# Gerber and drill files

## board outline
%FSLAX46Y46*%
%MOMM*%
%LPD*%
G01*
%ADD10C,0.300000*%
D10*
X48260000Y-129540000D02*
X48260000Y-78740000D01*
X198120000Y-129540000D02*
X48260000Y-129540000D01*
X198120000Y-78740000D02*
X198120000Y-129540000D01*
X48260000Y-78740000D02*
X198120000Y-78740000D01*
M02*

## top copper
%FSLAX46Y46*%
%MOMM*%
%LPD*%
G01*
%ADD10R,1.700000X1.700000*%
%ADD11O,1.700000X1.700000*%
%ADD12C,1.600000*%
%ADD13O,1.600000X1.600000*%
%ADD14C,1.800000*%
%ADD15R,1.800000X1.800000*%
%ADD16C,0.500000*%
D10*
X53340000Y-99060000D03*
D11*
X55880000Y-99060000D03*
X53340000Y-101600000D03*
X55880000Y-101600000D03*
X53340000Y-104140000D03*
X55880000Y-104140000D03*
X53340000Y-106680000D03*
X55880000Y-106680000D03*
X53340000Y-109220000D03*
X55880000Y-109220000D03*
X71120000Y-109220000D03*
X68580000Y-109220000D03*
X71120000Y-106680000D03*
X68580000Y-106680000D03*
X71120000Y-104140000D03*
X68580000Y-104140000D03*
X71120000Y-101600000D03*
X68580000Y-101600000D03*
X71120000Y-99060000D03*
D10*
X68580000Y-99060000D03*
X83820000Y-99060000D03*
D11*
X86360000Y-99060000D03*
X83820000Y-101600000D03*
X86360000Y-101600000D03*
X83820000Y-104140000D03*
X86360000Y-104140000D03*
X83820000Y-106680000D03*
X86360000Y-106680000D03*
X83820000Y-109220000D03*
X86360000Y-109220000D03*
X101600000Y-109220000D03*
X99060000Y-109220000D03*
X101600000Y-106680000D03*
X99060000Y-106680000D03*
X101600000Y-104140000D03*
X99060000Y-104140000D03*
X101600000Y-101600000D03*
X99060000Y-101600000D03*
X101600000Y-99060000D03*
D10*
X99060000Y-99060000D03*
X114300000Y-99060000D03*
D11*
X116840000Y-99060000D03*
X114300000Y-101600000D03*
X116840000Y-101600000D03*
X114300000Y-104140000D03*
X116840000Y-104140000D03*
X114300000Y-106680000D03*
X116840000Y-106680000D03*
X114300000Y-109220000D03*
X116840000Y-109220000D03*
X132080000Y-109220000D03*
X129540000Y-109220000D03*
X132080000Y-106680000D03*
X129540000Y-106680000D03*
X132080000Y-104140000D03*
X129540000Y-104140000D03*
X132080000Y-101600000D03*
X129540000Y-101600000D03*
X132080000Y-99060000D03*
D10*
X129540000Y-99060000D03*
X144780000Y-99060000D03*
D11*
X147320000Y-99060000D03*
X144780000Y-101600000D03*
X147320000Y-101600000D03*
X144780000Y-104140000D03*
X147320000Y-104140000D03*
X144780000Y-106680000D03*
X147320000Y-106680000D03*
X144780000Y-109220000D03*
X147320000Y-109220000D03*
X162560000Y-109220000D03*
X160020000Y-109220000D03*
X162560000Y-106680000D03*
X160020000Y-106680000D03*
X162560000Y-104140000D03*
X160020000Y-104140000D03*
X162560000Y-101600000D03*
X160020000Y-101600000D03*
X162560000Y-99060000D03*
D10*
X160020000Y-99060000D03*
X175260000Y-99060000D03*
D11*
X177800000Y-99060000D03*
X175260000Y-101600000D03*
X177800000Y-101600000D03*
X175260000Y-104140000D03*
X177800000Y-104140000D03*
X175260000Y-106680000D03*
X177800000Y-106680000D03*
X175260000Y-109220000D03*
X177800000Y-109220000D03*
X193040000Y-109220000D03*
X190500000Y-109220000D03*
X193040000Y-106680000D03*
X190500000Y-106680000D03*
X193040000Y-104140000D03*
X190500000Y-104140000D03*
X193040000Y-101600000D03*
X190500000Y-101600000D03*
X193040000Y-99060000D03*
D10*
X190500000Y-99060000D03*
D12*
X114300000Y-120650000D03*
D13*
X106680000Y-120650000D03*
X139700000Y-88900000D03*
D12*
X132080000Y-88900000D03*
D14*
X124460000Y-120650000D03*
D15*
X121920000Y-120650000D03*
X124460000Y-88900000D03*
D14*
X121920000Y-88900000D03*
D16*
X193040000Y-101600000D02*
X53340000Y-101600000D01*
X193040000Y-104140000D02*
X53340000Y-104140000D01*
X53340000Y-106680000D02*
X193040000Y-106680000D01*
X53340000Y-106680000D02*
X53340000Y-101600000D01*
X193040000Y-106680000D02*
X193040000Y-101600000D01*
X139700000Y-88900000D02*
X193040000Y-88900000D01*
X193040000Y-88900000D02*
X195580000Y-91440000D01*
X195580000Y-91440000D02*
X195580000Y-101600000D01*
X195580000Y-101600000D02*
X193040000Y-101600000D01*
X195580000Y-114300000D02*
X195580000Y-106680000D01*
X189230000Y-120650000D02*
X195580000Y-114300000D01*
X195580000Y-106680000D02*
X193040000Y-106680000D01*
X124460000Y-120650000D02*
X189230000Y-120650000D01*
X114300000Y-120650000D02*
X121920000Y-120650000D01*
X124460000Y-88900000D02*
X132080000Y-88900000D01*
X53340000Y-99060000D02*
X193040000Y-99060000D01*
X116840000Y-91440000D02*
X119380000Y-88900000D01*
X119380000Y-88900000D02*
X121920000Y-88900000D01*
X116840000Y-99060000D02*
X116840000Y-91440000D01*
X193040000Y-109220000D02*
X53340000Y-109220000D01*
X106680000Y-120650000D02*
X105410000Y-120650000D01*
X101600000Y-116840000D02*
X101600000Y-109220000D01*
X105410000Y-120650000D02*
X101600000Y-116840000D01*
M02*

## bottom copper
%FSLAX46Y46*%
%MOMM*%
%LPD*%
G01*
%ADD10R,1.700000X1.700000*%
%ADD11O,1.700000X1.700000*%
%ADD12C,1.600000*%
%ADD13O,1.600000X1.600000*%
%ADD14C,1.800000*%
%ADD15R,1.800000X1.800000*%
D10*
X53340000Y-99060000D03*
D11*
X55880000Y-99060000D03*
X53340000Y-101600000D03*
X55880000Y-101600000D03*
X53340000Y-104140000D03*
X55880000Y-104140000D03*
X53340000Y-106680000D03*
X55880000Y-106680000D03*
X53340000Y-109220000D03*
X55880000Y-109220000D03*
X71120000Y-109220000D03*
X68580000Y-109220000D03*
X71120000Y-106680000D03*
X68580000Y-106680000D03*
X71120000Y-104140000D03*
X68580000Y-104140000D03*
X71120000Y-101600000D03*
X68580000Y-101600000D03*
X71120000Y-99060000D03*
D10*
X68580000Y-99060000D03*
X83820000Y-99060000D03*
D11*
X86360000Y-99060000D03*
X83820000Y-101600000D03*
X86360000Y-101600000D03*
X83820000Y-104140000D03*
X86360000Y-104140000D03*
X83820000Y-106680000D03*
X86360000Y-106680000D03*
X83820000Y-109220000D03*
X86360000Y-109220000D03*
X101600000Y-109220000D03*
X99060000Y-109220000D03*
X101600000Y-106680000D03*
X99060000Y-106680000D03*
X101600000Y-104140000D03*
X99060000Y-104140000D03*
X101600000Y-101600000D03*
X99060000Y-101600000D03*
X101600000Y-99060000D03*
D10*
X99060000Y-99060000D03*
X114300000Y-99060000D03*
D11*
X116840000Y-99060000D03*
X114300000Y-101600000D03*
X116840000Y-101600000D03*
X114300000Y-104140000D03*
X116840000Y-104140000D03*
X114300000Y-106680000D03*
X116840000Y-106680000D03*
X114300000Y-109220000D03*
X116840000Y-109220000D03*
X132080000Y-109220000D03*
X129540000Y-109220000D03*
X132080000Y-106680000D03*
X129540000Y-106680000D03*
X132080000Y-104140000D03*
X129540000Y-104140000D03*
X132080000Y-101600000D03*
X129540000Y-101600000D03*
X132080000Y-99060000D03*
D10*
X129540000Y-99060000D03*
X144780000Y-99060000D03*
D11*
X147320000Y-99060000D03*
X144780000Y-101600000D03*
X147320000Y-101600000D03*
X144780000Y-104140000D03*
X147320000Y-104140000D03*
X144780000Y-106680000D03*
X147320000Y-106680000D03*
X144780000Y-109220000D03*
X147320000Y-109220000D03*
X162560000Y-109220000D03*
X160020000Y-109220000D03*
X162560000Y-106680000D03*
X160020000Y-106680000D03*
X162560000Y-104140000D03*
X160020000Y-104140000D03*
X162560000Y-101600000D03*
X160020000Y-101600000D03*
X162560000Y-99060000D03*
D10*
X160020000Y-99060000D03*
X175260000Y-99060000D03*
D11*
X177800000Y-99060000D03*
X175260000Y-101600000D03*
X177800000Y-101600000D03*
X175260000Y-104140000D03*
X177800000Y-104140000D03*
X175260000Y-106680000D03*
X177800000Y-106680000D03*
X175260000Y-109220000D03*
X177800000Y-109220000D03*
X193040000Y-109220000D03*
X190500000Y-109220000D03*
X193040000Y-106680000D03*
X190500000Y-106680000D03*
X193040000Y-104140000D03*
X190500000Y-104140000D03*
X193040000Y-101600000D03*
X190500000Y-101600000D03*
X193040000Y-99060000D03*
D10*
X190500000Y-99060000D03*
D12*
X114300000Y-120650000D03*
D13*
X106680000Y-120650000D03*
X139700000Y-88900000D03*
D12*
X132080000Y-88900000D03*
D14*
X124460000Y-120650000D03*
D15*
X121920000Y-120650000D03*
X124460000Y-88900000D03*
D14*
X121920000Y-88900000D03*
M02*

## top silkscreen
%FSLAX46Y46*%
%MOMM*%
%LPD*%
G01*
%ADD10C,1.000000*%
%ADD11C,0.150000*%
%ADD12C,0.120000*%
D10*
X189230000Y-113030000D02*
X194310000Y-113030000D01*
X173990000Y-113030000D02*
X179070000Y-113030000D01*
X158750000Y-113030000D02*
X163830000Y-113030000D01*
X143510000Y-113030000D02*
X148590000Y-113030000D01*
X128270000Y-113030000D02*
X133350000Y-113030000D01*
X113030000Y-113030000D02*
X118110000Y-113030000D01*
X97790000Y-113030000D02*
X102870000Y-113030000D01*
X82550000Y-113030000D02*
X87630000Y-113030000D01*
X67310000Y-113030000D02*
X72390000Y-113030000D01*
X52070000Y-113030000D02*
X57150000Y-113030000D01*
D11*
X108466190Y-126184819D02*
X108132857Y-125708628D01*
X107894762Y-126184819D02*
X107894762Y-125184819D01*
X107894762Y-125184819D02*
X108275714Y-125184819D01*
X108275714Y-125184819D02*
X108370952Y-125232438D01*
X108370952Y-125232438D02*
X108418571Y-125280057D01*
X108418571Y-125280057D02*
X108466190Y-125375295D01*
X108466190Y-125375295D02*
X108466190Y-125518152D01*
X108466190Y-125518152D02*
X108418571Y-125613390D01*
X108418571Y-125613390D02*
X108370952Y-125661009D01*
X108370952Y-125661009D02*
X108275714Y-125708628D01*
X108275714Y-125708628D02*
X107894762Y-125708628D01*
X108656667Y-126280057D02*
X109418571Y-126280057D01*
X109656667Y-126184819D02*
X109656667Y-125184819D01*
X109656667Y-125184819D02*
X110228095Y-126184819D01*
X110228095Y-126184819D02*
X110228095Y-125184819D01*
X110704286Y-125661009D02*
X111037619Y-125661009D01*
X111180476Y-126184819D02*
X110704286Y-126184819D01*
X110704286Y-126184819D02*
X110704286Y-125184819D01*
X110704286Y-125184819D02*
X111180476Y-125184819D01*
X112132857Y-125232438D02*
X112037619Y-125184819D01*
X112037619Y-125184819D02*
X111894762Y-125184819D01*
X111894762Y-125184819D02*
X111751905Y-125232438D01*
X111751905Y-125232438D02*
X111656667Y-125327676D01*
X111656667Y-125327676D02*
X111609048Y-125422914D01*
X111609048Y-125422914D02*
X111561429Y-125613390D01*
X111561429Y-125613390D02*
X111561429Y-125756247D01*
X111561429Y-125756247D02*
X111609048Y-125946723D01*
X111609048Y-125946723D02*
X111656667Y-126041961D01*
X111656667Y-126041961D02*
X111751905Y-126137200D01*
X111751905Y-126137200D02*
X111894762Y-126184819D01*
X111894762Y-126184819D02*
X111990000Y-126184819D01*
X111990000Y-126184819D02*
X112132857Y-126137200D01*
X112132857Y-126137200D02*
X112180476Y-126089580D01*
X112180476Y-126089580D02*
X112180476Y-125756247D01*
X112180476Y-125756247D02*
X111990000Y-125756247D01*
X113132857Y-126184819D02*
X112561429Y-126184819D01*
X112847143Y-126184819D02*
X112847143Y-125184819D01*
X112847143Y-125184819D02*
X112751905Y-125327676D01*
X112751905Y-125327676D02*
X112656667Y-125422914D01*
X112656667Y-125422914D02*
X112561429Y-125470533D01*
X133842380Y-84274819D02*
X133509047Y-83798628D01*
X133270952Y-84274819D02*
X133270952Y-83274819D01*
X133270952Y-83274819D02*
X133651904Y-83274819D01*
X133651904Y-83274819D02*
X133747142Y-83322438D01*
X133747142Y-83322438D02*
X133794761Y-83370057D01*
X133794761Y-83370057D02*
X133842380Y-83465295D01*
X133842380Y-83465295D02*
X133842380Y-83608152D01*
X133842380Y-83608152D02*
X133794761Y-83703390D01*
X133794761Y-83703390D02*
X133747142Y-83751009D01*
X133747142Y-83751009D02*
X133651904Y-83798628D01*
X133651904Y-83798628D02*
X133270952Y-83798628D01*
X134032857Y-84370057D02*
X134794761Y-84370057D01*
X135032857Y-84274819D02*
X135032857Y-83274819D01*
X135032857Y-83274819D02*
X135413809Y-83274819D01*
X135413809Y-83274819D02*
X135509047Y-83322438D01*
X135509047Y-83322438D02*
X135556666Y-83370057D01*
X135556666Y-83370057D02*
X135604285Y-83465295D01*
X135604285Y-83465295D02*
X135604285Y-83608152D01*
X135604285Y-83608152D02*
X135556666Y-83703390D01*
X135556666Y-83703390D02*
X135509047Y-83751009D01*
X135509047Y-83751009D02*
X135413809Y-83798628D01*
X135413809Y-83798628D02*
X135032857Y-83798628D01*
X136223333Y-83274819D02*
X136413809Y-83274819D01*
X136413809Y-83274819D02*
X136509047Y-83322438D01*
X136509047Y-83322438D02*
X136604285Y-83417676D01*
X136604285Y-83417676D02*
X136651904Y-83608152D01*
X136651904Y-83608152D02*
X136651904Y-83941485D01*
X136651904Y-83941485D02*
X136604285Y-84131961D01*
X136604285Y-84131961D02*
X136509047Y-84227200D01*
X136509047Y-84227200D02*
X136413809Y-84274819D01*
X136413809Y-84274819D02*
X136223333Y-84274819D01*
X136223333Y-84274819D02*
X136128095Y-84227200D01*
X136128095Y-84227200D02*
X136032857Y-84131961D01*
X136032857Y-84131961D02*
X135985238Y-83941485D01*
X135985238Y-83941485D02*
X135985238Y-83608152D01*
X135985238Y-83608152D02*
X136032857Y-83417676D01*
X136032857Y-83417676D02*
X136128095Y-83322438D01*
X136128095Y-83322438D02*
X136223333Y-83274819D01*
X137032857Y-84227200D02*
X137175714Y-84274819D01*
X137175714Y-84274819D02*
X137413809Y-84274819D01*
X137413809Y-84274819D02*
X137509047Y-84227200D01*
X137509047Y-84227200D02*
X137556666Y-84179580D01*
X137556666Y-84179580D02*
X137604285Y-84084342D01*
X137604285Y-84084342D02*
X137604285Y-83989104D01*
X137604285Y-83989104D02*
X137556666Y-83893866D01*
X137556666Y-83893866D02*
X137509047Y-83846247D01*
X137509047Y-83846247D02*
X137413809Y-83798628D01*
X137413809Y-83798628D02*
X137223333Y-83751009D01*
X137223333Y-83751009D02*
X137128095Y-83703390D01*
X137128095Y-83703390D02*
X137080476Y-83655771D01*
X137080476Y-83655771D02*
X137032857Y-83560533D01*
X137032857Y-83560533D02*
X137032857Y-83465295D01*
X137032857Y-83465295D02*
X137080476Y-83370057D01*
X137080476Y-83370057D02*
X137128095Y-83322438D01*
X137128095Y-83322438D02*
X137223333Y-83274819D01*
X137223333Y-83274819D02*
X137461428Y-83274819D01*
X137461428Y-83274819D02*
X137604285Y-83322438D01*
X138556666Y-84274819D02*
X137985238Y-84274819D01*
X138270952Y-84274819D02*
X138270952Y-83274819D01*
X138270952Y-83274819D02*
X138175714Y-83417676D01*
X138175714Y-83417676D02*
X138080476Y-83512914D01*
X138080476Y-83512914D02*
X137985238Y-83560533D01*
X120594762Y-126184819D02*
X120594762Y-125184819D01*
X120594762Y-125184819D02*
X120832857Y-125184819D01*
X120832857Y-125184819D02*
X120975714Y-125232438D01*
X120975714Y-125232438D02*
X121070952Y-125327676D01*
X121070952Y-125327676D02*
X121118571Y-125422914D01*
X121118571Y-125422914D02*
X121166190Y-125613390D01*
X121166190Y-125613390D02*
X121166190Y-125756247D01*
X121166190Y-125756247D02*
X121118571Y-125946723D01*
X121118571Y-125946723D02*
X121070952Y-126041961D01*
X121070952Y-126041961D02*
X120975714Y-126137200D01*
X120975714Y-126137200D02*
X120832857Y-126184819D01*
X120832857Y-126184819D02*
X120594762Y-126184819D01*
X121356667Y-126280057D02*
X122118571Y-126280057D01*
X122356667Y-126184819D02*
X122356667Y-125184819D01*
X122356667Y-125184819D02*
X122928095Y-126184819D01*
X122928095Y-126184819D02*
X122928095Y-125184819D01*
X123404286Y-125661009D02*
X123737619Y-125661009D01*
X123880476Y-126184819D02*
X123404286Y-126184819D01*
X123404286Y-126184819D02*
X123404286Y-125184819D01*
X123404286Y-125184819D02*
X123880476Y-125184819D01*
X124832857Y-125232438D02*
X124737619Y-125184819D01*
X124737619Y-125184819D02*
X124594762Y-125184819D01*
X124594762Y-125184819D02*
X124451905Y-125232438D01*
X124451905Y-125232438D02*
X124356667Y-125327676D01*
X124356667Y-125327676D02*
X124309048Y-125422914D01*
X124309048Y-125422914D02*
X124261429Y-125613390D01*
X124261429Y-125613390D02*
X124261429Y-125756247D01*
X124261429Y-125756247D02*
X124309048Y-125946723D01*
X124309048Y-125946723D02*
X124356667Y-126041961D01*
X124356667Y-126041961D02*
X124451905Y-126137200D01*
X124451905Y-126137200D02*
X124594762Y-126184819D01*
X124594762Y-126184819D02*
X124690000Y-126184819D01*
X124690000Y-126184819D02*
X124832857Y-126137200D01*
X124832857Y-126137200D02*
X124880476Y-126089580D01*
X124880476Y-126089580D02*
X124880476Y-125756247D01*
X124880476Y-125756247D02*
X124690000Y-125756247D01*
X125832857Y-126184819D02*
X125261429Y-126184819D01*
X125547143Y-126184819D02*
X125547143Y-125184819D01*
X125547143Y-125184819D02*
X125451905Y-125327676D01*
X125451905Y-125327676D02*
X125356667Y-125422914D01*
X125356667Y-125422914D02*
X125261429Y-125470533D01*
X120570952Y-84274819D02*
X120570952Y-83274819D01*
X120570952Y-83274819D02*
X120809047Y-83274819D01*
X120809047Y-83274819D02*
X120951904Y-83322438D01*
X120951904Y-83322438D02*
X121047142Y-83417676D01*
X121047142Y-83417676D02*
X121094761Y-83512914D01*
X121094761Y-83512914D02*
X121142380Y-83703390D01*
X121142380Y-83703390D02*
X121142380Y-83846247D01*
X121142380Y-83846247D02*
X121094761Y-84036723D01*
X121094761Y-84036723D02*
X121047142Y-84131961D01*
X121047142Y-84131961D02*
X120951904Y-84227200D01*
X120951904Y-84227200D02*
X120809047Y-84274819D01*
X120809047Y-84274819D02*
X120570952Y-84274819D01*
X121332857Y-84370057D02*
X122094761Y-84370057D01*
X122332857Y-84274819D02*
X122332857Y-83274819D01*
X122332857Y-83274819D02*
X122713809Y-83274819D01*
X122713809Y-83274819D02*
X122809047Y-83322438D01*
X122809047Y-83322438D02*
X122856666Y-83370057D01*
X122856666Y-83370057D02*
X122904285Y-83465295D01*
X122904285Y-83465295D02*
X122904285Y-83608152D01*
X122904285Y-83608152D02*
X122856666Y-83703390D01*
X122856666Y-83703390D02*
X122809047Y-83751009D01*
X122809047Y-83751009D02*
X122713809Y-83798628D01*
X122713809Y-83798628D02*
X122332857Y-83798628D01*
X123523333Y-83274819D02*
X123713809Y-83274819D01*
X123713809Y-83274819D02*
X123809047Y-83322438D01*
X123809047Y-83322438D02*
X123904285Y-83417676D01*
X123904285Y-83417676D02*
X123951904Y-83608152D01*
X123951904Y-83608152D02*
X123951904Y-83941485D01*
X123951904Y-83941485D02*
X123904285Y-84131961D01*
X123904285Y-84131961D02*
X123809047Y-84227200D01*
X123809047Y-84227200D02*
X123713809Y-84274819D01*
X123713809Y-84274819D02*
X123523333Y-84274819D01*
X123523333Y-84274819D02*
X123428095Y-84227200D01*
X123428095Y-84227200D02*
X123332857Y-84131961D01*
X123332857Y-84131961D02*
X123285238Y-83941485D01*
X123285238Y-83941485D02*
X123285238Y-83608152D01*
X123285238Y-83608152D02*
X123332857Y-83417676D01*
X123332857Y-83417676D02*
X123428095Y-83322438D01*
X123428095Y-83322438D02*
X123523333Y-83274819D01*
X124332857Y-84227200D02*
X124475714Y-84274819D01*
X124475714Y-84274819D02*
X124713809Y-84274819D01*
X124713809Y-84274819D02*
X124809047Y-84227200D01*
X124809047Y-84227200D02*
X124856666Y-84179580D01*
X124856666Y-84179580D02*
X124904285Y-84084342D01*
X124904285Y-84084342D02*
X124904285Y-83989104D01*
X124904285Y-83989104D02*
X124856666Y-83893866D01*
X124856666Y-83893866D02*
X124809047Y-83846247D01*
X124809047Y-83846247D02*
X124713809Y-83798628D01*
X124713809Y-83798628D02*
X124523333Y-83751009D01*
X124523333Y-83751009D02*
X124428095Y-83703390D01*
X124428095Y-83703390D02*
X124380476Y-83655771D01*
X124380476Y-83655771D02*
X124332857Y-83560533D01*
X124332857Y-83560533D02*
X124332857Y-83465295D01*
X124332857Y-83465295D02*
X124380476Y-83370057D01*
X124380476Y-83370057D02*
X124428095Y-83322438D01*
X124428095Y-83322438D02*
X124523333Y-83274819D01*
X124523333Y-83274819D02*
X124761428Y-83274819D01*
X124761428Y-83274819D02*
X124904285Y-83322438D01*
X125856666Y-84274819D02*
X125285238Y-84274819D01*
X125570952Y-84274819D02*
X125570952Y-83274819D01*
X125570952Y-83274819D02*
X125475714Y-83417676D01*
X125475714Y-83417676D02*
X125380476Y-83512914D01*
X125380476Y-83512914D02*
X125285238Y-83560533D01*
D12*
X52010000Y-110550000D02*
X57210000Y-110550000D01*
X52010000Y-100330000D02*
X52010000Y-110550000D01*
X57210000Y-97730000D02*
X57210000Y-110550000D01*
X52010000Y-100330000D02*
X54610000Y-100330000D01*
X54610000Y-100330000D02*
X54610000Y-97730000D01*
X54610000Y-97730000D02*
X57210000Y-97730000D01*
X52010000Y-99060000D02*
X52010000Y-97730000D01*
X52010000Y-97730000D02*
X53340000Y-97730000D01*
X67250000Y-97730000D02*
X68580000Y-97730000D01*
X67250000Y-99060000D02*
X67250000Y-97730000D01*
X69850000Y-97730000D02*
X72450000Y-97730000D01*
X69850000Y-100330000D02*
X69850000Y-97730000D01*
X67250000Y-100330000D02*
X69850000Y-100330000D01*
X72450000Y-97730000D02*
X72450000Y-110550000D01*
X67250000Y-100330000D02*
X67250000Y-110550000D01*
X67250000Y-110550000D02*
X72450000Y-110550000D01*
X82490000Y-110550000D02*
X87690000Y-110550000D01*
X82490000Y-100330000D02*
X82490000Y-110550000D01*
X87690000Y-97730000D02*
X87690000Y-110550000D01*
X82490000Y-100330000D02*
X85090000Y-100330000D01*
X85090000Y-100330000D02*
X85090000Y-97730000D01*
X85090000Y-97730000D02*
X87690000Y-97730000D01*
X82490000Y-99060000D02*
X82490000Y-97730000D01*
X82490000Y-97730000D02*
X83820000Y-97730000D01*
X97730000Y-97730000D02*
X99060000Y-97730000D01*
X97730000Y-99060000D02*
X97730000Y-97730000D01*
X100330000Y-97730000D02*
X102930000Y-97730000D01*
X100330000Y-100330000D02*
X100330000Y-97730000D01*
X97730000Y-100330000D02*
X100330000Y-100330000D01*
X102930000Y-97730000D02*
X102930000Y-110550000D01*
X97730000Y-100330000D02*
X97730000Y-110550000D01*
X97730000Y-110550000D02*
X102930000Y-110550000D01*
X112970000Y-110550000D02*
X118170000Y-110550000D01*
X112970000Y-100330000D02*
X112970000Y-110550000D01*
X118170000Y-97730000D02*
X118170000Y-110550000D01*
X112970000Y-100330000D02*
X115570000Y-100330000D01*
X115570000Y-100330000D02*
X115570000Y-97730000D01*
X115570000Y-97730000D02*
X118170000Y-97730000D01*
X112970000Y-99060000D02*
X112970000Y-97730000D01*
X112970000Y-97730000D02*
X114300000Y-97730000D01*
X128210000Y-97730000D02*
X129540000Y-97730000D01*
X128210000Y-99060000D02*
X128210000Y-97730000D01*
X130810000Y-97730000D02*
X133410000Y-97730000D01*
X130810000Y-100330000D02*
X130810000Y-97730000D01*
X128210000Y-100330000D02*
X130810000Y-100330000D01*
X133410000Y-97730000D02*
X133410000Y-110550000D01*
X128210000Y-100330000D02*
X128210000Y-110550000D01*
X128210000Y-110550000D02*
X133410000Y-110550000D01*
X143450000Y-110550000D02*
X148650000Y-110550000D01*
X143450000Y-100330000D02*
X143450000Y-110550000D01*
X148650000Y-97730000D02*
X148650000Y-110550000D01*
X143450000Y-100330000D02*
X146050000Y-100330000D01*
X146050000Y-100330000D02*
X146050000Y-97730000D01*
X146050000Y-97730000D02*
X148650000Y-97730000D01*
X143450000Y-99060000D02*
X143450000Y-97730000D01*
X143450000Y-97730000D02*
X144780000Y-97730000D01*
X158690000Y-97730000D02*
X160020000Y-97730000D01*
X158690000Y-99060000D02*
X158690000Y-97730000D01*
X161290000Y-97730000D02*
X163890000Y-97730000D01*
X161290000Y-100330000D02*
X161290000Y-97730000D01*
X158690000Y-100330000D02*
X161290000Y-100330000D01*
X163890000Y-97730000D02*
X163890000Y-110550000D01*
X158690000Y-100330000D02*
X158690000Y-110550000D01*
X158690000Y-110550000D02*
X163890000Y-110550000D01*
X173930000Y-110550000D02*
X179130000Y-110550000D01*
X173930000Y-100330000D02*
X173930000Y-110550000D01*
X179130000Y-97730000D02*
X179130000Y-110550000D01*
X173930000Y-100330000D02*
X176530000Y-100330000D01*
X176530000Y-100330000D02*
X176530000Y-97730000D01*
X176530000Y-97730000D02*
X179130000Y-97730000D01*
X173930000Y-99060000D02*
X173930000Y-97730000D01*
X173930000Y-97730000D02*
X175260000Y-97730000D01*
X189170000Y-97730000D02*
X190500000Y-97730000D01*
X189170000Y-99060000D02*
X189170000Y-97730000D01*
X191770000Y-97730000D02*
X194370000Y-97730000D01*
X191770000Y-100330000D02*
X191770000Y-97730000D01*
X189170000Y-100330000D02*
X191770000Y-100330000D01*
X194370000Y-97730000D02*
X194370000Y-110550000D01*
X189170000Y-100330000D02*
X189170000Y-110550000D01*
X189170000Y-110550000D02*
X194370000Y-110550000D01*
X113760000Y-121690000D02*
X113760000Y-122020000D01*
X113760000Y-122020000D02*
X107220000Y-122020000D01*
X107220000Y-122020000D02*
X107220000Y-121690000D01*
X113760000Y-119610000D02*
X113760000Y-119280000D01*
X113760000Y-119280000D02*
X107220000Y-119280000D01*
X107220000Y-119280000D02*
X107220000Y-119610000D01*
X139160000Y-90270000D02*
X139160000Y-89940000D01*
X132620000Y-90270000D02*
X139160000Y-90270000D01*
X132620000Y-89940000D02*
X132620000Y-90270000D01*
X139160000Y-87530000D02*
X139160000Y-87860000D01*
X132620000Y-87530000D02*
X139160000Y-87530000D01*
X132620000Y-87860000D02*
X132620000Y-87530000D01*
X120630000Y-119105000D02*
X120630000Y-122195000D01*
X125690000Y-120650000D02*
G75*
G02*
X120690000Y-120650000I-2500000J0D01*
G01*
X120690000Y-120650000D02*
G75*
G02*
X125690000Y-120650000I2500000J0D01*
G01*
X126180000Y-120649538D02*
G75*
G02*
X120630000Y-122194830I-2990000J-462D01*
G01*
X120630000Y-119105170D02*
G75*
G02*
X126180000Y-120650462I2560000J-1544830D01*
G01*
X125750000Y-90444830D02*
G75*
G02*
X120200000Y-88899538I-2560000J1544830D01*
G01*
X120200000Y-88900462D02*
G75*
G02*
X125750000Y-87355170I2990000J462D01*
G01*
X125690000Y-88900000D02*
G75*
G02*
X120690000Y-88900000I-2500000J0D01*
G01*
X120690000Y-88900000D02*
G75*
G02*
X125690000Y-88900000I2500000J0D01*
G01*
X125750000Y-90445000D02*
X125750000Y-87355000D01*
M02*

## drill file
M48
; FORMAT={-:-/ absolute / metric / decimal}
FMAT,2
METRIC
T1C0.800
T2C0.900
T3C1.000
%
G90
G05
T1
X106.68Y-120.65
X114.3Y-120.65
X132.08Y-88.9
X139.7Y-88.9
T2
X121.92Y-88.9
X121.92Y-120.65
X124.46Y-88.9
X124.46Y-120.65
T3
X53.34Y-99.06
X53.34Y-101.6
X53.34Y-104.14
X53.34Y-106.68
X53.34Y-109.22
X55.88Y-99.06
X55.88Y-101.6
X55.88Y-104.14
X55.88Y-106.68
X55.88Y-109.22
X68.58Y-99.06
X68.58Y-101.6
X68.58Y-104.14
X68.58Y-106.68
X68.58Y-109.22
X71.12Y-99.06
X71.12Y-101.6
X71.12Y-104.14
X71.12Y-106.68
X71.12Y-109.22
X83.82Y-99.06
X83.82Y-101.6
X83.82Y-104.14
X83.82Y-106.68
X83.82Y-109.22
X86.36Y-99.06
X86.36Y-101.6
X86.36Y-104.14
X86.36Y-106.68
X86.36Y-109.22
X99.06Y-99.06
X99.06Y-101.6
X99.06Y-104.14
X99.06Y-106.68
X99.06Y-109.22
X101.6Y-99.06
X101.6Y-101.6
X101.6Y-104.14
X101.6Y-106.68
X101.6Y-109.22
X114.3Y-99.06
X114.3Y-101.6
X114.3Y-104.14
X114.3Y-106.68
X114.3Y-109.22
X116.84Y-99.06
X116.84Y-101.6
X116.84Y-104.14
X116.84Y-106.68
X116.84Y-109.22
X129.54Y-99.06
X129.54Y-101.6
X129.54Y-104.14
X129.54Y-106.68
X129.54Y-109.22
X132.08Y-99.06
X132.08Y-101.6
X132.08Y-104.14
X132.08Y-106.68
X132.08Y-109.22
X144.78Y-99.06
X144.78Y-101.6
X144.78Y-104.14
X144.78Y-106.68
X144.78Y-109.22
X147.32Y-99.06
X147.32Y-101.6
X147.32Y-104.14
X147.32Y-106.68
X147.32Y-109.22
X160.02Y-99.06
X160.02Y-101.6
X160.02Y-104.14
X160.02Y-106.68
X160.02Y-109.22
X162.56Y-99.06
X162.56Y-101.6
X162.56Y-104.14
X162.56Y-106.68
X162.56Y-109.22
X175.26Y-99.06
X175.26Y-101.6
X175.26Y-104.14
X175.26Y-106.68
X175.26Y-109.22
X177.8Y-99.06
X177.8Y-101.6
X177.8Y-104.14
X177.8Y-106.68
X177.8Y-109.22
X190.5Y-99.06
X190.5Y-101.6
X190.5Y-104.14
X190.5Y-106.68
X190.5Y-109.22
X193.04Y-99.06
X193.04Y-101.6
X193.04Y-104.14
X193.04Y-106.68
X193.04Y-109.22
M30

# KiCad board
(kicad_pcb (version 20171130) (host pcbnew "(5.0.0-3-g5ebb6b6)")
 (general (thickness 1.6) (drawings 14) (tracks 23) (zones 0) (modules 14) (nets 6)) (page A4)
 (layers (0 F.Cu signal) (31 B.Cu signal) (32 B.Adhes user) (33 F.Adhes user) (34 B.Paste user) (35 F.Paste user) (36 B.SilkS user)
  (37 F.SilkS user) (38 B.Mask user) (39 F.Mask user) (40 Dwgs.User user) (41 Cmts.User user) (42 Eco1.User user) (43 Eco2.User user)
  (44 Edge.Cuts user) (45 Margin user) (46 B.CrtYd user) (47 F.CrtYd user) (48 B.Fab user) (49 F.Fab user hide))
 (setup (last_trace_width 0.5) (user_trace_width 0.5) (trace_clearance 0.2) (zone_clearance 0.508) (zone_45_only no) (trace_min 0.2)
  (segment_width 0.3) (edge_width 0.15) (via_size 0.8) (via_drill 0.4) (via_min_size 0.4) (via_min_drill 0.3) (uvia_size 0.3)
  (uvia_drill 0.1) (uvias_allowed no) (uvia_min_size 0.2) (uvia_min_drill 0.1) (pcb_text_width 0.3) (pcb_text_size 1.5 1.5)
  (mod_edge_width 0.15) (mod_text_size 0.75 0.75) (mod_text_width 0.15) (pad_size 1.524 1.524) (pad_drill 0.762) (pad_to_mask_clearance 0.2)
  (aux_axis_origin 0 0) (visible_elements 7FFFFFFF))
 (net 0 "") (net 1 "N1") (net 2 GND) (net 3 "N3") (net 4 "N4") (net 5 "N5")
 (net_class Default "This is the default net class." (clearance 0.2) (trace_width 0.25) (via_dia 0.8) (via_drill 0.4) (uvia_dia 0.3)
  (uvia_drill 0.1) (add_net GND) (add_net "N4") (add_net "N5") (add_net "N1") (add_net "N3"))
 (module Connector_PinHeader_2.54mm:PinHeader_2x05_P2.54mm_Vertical (layer F.Cu) (at 53.34 99.06)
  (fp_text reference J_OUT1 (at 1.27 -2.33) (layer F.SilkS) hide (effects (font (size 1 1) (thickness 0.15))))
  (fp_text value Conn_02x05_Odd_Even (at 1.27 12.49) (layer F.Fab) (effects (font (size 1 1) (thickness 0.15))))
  (fp_line (start -1.33 11.49) (end 3.87 11.49) (layer F.SilkS) (width 0.12))
  (fp_line (start -1.33 1.27) (end -1.33 11.49) (layer F.SilkS) (width 0.12))
  (fp_line (start 3.87 -1.33) (end 3.87 11.49) (layer F.SilkS) (width 0.12))
  (fp_line (start -1.33 1.27) (end 1.27 1.27) (layer F.SilkS) (width 0.12))
  (fp_line (start 1.27 1.27) (end 1.27 -1.33) (layer F.SilkS) (width 0.12))
  (fp_line (start 1.27 -1.33) (end 3.87 -1.33) (layer F.SilkS) (width 0.12))
  (fp_line (start -1.33 0) (end -1.33 -1.33) (layer F.SilkS) (width 0.12))
  (fp_line (start -1.33 -1.33) (end 0 -1.33) (layer F.SilkS) (width 0.12))
  (pad 1 thru_hole rect (at 0 0) (size 1.7 1.7) (drill 1) (layers *.Cu *.Mask) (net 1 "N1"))
  (pad 2 thru_hole oval (at 2.54 0) (size 1.7 1.7) (drill 1) (layers *.Cu *.Mask) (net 1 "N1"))
  (pad 3 thru_hole oval (at 0 2.54) (size 1.7 1.7) (drill 1) (layers *.Cu *.Mask) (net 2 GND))
  (pad 4 thru_hole oval (at 2.54 2.54) (size 1.7 1.7) (drill 1) (layers *.Cu *.Mask) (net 2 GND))
  (pad 5 thru_hole oval (at 0 5.08) (size 1.7 1.7) (drill 1) (layers *.Cu *.Mask) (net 2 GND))
  (pad 6 thru_hole oval (at 2.54 5.08) (size 1.7 1.7) (drill 1) (layers *.Cu *.Mask) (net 2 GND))
  (pad 7 thru_hole oval (at 0 7.62) (size 1.7 1.7) (drill 1) (layers *.Cu *.Mask) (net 2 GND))
  (pad 8 thru_hole oval (at 2.54 7.62) (size 1.7 1.7) (drill 1) (layers *.Cu *.Mask) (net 2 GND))
  (pad 9 thru_hole oval (at 0 10.16) (size 1.7 1.7) (drill 1) (layers *.Cu *.Mask) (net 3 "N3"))
  (pad 10 thru_hole oval (at 2.54 10.16) (size 1.7 1.7) (drill 1) (layers *.Cu *.Mask) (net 3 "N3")))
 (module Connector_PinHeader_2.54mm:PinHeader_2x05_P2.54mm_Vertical (layer F.Cu) (at 68.58 99.06)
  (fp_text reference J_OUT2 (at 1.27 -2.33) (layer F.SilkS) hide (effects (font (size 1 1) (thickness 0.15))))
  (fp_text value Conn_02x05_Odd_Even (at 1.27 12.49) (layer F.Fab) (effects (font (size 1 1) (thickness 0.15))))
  (fp_line (start -1.33 -1.33) (end 0 -1.33) (layer F.SilkS) (width 0.12))
  (fp_line (start -1.33 0) (end -1.33 -1.33) (layer F.SilkS) (width 0.12))
  (fp_line (start 1.27 -1.33) (end 3.87 -1.33) (layer F.SilkS) (width 0.12))
  (fp_line (start 1.27 1.27) (end 1.27 -1.33) (layer F.SilkS) (width 0.12))
  (fp_line (start -1.33 1.27) (end 1.27 1.27) (layer F.SilkS) (width 0.12))
  (fp_line (start 3.87 -1.33) (end 3.87 11.49) (layer F.SilkS) (width 0.12))
  (fp_line (start -1.33 1.27) (end -1.33 11.49) (layer F.SilkS) (width 0.12))
  (fp_line (start -1.33 11.49) (end 3.87 11.49) (layer F.SilkS) (width 0.12))
  (pad 10 thru_hole oval (at 2.54 10.16) (size 1.7 1.7) (drill 1) (layers *.Cu *.Mask) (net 3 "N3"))
  (pad 9 thru_hole oval (at 0 10.16) (size 1.7 1.7) (drill 1) (layers *.Cu *.Mask) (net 3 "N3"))
  (pad 8 thru_hole oval (at 2.54 7.62) (size 1.7 1.7) (drill 1) (layers *.Cu *.Mask) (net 2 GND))
  (pad 7 thru_hole oval (at 0 7.62) (size 1.7 1.7) (drill 1) (layers *.Cu *.Mask) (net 2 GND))
  (pad 6 thru_hole oval (at 2.54 5.08) (size 1.7 1.7) (drill 1) (layers *.Cu *.Mask) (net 2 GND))
  (pad 5 thru_hole oval (at 0 5.08) (size 1.7 1.7) (drill 1) (layers *.Cu *.Mask) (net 2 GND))
  (pad 4 thru_hole oval (at 2.54 2.54) (size 1.7 1.7) (drill 1) (layers *.Cu *.Mask) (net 2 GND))
  (pad 3 thru_hole oval (at 0 2.54) (size 1.7 1.7) (drill 1) (layers *.Cu *.Mask) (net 2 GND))
  (pad 2 thru_hole oval (at 2.54 0) (size 1.7 1.7) (drill 1) (layers *.Cu *.Mask) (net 1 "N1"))
  (pad 1 thru_hole rect (at 0 0) (size 1.7 1.7) (drill 1) (layers *.Cu *.Mask) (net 1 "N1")))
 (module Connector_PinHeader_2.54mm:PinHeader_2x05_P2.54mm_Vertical (layer F.Cu) (at 83.82 99.06)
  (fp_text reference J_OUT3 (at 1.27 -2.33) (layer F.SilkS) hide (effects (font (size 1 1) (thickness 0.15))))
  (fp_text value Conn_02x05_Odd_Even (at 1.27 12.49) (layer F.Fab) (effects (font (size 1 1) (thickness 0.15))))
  (fp_line (start -1.33 11.49) (end 3.87 11.49) (layer F.SilkS) (width 0.12))
  (fp_line (start -1.33 1.27) (end -1.33 11.49) (layer F.SilkS) (width 0.12))
  (fp_line (start 3.87 -1.33) (end 3.87 11.49) (layer F.SilkS) (width 0.12))
  (fp_line (start -1.33 1.27) (end 1.27 1.27) (layer F.SilkS) (width 0.12))
  (fp_line (start 1.27 1.27) (end 1.27 -1.33) (layer F.SilkS) (width 0.12))
  (fp_line (start 1.27 -1.33) (end 3.87 -1.33) (layer F.SilkS) (width 0.12))
  (fp_line (start -1.33 0) (end -1.33 -1.33) (layer F.SilkS) (width 0.12))
  (fp_line (start -1.33 -1.33) (end 0 -1.33) (layer F.SilkS) (width 0.12))
  (pad 1 thru_hole rect (at 0 0) (size 1.7 1.7) (drill 1) (layers *.Cu *.Mask) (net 1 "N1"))
  (pad 2 thru_hole oval (at 2.54 0) (size 1.7 1.7) (drill 1) (layers *.Cu *.Mask) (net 1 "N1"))
  (pad 3 thru_hole oval (at 0 2.54) (size 1.7 1.7) (drill 1) (layers *.Cu *.Mask) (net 2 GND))
  (pad 4 thru_hole oval (at 2.54 2.54) (size 1.7 1.7) (drill 1) (layers *.Cu *.Mask) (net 2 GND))
  (pad 5 thru_hole oval (at 0 5.08) (size 1.7 1.7) (drill 1) (layers *.Cu *.Mask) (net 2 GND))
  (pad 6 thru_hole oval (at 2.54 5.08) (size 1.7 1.7) (drill 1) (layers *.Cu *.Mask) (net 2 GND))
  (pad 7 thru_hole oval (at 0 7.62) (size 1.7 1.7) (drill 1) (layers *.Cu *.Mask) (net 2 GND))
  (pad 8 thru_hole oval (at 2.54 7.62) (size 1.7 1.7) (drill 1) (layers *.Cu *.Mask) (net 2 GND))
  (pad 9 thru_hole oval (at 0 10.16) (size 1.7 1.7) (drill 1) (layers *.Cu *.Mask) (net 3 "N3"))
  (pad 10 thru_hole oval (at 2.54 10.16) (size 1.7 1.7) (drill 1) (layers *.Cu *.Mask) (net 3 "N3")))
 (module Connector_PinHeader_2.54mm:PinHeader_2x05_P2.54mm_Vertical (layer F.Cu) (at 99.06 99.06)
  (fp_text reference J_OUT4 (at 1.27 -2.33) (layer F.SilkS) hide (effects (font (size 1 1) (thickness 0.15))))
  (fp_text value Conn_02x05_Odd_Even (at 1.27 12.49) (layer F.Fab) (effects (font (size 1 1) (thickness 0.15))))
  (fp_line (start -1.33 -1.33) (end 0 -1.33) (layer F.SilkS) (width 0.12))
  (fp_line (start -1.33 0) (end -1.33 -1.33) (layer F.SilkS) (width 0.12))
  (fp_line (start 1.27 -1.33) (end 3.87 -1.33) (layer F.SilkS) (width 0.12))
  (fp_line (start 1.27 1.27) (end 1.27 -1.33) (layer F.SilkS) (width 0.12))
  (fp_line (start -1.33 1.27) (end 1.27 1.27) (layer F.SilkS) (width 0.12))
  (fp_line (start 3.87 -1.33) (end 3.87 11.49) (layer F.SilkS) (width 0.12))
  (fp_line (start -1.33 1.27) (end -1.33 11.49) (layer F.SilkS) (width 0.12))
  (fp_line (start -1.33 11.49) (end 3.87 11.49) (layer F.SilkS) (width 0.12))
  (pad 10 thru_hole oval (at 2.54 10.16) (size 1.7 1.7) (drill 1) (layers *.Cu *.Mask) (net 3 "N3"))
  (pad 9 thru_hole oval (at 0 10.16) (size 1.7 1.7) (drill 1) (layers *.Cu *.Mask) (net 3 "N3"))
  (pad 8 thru_hole oval (at 2.54 7.62) (size 1.7 1.7) (drill 1) (layers *.Cu *.Mask) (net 2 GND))
  (pad 7 thru_hole oval (at 0 7.62) (size 1.7 1.7) (drill 1) (layers *.Cu *.Mask) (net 2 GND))
  (pad 6 thru_hole oval (at 2.54 5.08) (size 1.7 1.7) (drill 1) (layers *.Cu *.Mask) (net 2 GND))
  (pad 5 thru_hole oval (at 0 5.08) (size 1.7 1.7) (drill 1) (layers *.Cu *.Mask) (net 2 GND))
  (pad 4 thru_hole oval (at 2.54 2.54) (size 1.7 1.7) (drill 1) (layers *.Cu *.Mask) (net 2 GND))
  (pad 3 thru_hole oval (at 0 2.54) (size 1.7 1.7) (drill 1) (layers *.Cu *.Mask) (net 2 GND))
  (pad 2 thru_hole oval (at 2.54 0) (size 1.7 1.7) (drill 1) (layers *.Cu *.Mask) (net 1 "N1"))
  (pad 1 thru_hole rect (at 0 0) (size 1.7 1.7) (drill 1) (layers *.Cu *.Mask) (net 1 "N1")))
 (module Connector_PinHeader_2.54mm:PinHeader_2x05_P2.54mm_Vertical (layer F.Cu) (at 114.3 99.06)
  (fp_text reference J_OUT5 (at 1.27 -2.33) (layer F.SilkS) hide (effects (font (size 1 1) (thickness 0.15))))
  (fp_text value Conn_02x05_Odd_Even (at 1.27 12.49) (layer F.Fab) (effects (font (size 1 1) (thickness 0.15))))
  (fp_line (start -1.33 11.49) (end 3.87 11.49) (layer F.SilkS) (width 0.12))
  (fp_line (start -1.33 1.27) (end -1.33 11.49) (layer F.SilkS) (width 0.12))
  (fp_line (start 3.87 -1.33) (end 3.87 11.49) (layer F.SilkS) (width 0.12))
  (fp_line (start -1.33 1.27) (end 1.27 1.27) (layer F.SilkS) (width 0.12))
  (fp_line (start 1.27 1.27) (end 1.27 -1.33) (layer F.SilkS) (width 0.12))
  (fp_line (start 1.27 -1.33) (end 3.87 -1.33) (layer F.SilkS) (width 0.12))
  (fp_line (start -1.33 0) (end -1.33 -1.33) (layer F.SilkS) (width 0.12))
  (fp_line (start -1.33 -1.33) (end 0 -1.33) (layer F.SilkS) (width 0.12))
  (pad 1 thru_hole rect (at 0 0) (size 1.7 1.7) (drill 1) (layers *.Cu *.Mask) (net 1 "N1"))
  (pad 2 thru_hole oval (at 2.54 0) (size 1.7 1.7) (drill 1) (layers *.Cu *.Mask) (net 1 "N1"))
  (pad 3 thru_hole oval (at 0 2.54) (size 1.7 1.7) (drill 1) (layers *.Cu *.Mask) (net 2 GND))
  (pad 4 thru_hole oval (at 2.54 2.54) (size 1.7 1.7) (drill 1) (layers *.Cu *.Mask) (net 2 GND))
  (pad 5 thru_hole oval (at 0 5.08) (size 1.7 1.7) (drill 1) (layers *.Cu *.Mask) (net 2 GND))
  (pad 6 thru_hole oval (at 2.54 5.08) (size 1.7 1.7) (drill 1) (layers *.Cu *.Mask) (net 2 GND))
  (pad 7 thru_hole oval (at 0 7.62) (size 1.7 1.7) (drill 1) (layers *.Cu *.Mask) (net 2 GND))
  (pad 8 thru_hole oval (at 2.54 7.62) (size 1.7 1.7) (drill 1) (layers *.Cu *.Mask) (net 2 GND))
  (pad 9 thru_hole oval (at 0 10.16) (size 1.7 1.7) (drill 1) (layers *.Cu *.Mask) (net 3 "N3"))
  (pad 10 thru_hole oval (at 2.54 10.16) (size 1.7 1.7) (drill 1) (layers *.Cu *.Mask) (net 3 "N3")))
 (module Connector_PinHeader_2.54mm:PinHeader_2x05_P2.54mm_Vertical (layer F.Cu) (at 129.54 99.06)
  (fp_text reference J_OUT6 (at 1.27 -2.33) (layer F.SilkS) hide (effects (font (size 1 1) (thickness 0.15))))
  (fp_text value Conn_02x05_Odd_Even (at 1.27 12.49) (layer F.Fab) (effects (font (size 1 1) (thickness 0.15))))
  (fp_line (start -1.33 -1.33) (end 0 -1.33) (layer F.SilkS) (width 0.12))
  (fp_line (start -1.33 0) (end -1.33 -1.33) (layer F.SilkS) (width 0.12))
  (fp_line (start 1.27 -1.33) (end 3.87 -1.33) (layer F.SilkS) (width 0.12))
  (fp_line (start 1.27 1.27) (end 1.27 -1.33) (layer F.SilkS) (width 0.12))
  (fp_line (start -1.33 1.27) (end 1.27 1.27) (layer F.SilkS) (width 0.12))
  (fp_line (start 3.87 -1.33) (end 3.87 11.49) (layer F.SilkS) (width 0.12))
  (fp_line (start -1.33 1.27) (end -1.33 11.49) (layer F.SilkS) (width 0.12))
  (fp_line (start -1.33 11.49) (end 3.87 11.49) (layer F.SilkS) (width 0.12))
  (pad 10 thru_hole oval (at 2.54 10.16) (size 1.7 1.7) (drill 1) (layers *.Cu *.Mask) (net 3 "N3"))
  (pad 9 thru_hole oval (at 0 10.16) (size 1.7 1.7) (drill 1) (layers *.Cu *.Mask) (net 3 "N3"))
  (pad 8 thru_hole oval (at 2.54 7.62) (size 1.7 1.7) (drill 1) (layers *.Cu *.Mask) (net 2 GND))
  (pad 7 thru_hole oval (at 0 7.62) (size 1.7 1.7) (drill 1) (layers *.Cu *.Mask) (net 2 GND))
  (pad 6 thru_hole oval (at 2.54 5.08) (size 1.7 1.7) (drill 1) (layers *.Cu *.Mask) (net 2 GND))
  (pad 5 thru_hole oval (at 0 5.08) (size 1.7 1.7) (drill 1) (layers *.Cu *.Mask) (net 2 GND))
  (pad 4 thru_hole oval (at 2.54 2.54) (size 1.7 1.7) (drill 1) (layers *.Cu *.Mask) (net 2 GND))
  (pad 3 thru_hole oval (at 0 2.54) (size 1.7 1.7) (drill 1) (layers *.Cu *.Mask) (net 2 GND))
  (pad 2 thru_hole oval (at 2.54 0) (size 1.7 1.7) (drill 1) (layers *.Cu *.Mask) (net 1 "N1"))
  (pad 1 thru_hole rect (at 0 0) (size 1.7 1.7) (drill 1) (layers *.Cu *.Mask) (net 1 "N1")))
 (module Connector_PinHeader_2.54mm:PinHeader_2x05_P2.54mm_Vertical (layer F.Cu) (at 144.78 99.06)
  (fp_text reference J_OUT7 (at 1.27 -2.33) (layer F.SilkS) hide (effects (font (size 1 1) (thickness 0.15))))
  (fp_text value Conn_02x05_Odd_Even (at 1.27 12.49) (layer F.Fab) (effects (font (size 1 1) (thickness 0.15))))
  (fp_line (start -1.33 11.49) (end 3.87 11.49) (layer F.SilkS) (width 0.12))
  (fp_line (start -1.33 1.27) (end -1.33 11.49) (layer F.SilkS) (width 0.12))
  (fp_line (start 3.87 -1.33) (end 3.87 11.49) (layer F.SilkS) (width 0.12))
  (fp_line (start -1.33 1.27) (end 1.27 1.27) (layer F.SilkS) (width 0.12))
  (fp_line (start 1.27 1.27) (end 1.27 -1.33) (layer F.SilkS) (width 0.12))
  (fp_line (start 1.27 -1.33) (end 3.87 -1.33) (layer F.SilkS) (width 0.12))
  (fp_line (start -1.33 0) (end -1.33 -1.33) (layer F.SilkS) (width 0.12))
  (fp_line (start -1.33 -1.33) (end 0 -1.33) (layer F.SilkS) (width 0.12))
  (pad 1 thru_hole rect (at 0 0) (size 1.7 1.7) (drill 1) (layers *.Cu *.Mask) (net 1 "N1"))
  (pad 2 thru_hole oval (at 2.54 0) (size 1.7 1.7) (drill 1) (layers *.Cu *.Mask) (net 1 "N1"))
  (pad 3 thru_hole oval (at 0 2.54) (size 1.7 1.7) (drill 1) (layers *.Cu *.Mask) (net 2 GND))
  (pad 4 thru_hole oval (at 2.54 2.54) (size 1.7 1.7) (drill 1) (layers *.Cu *.Mask) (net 2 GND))
  (pad 5 thru_hole oval (at 0 5.08) (size 1.7 1.7) (drill 1) (layers *.Cu *.Mask) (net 2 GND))
  (pad 6 thru_hole oval (at 2.54 5.08) (size 1.7 1.7) (drill 1) (layers *.Cu *.Mask) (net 2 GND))
  (pad 7 thru_hole oval (at 0 7.62) (size 1.7 1.7) (drill 1) (layers *.Cu *.Mask) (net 2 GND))
  (pad 8 thru_hole oval (at 2.54 7.62) (size 1.7 1.7) (drill 1) (layers *.Cu *.Mask) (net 2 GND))
  (pad 9 thru_hole oval (at 0 10.16) (size 1.7 1.7) (drill 1) (layers *.Cu *.Mask) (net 3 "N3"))
  (pad 10 thru_hole oval (at 2.54 10.16) (size 1.7 1.7) (drill 1) (layers *.Cu *.Mask) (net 3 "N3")))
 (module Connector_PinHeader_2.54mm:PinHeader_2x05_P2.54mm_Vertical (layer F.Cu) (at 160.02 99.06)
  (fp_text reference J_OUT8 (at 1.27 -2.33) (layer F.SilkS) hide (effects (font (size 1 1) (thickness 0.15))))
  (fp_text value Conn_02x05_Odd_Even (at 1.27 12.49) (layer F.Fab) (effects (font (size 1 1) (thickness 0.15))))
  (fp_line (start -1.33 -1.33) (end 0 -1.33) (layer F.SilkS) (width 0.12))
  (fp_line (start -1.33 0) (end -1.33 -1.33) (layer F.SilkS) (width 0.12))
  (fp_line (start 1.27 -1.33) (end 3.87 -1.33) (layer F.SilkS) (width 0.12))
  (fp_line (start 1.27 1.27) (end 1.27 -1.33) (layer F.SilkS) (width 0.12))
  (fp_line (start -1.33 1.27) (end 1.27 1.27) (layer F.SilkS) (width 0.12))
  (fp_line (start 3.87 -1.33) (end 3.87 11.49) (layer F.SilkS) (width 0.12))
  (fp_line (start -1.33 1.27) (end -1.33 11.49) (layer F.SilkS) (width 0.12))
  (fp_line (start -1.33 11.49) (end 3.87 11.49) (layer F.SilkS) (width 0.12))
  (pad 10 thru_hole oval (at 2.54 10.16) (size 1.7 1.7) (drill 1) (layers *.Cu *.Mask) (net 3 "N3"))
  (pad 9 thru_hole oval (at 0 10.16) (size 1.7 1.7) (drill 1) (layers *.Cu *.Mask) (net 3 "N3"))
  (pad 8 thru_hole oval (at 2.54 7.62) (size 1.7 1.7) (drill 1) (layers *.Cu *.Mask) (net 2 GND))
  (pad 7 thru_hole oval (at 0 7.62) (size 1.7 1.7) (drill 1) (layers *.Cu *.Mask) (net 2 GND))
  (pad 6 thru_hole oval (at 2.54 5.08) (size 1.7 1.7) (drill 1) (layers *.Cu *.Mask) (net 2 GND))
  (pad 5 thru_hole oval (at 0 5.08) (size 1.7 1.7) (drill 1) (layers *.Cu *.Mask) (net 2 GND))
  (pad 4 thru_hole oval (at 2.54 2.54) (size 1.7 1.7) (drill 1) (layers *.Cu *.Mask) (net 2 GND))
  (pad 3 thru_hole oval (at 0 2.54) (size 1.7 1.7) (drill 1) (layers *.Cu *.Mask) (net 2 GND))
  (pad 2 thru_hole oval (at 2.54 0) (size 1.7 1.7) (drill 1) (layers *.Cu *.Mask) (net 1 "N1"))
  (pad 1 thru_hole rect (at 0 0) (size 1.7 1.7) (drill 1) (layers *.Cu *.Mask) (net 1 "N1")))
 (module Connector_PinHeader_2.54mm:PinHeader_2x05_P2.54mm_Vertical (layer F.Cu) (at 175.26 99.06)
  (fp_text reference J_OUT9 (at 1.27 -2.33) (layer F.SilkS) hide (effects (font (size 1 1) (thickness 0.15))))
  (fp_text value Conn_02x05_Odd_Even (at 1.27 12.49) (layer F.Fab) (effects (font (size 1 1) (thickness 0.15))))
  (fp_line (start -1.33 11.49) (end 3.87 11.49) (layer F.SilkS) (width 0.12))
  (fp_line (start -1.33 1.27) (end -1.33 11.49) (layer F.SilkS) (width 0.12))
  (fp_line (start 3.87 -1.33) (end 3.87 11.49) (layer F.SilkS) (width 0.12))
  (fp_line (start -1.33 1.27) (end 1.27 1.27) (layer F.SilkS) (width 0.12))
  (fp_line (start 1.27 1.27) (end 1.27 -1.33) (layer F.SilkS) (width 0.12))
  (fp_line (start 1.27 -1.33) (end 3.87 -1.33) (layer F.SilkS) (width 0.12))
  (fp_line (start -1.33 0) (end -1.33 -1.33) (layer F.SilkS) (width 0.12))
  (fp_line (start -1.33 -1.33) (end 0 -1.33) (layer F.SilkS) (width 0.12))
  (pad 1 thru_hole rect (at 0 0) (size 1.7 1.7) (drill 1) (layers *.Cu *.Mask) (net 1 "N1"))
  (pad 2 thru_hole oval (at 2.54 0) (size 1.7 1.7) (drill 1) (layers *.Cu *.Mask) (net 1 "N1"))
  (pad 3 thru_hole oval (at 0 2.54) (size 1.7 1.7) (drill 1) (layers *.Cu *.Mask) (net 2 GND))
  (pad 4 thru_hole oval (at 2.54 2.54) (size 1.7 1.7) (drill 1) (layers *.Cu *.Mask) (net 2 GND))
  (pad 5 thru_hole oval (at 0 5.08) (size 1.7 1.7) (drill 1) (layers *.Cu *.Mask) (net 2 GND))
  (pad 6 thru_hole oval (at 2.54 5.08) (size 1.7 1.7) (drill 1) (layers *.Cu *.Mask) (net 2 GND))
  (pad 7 thru_hole oval (at 0 7.62) (size 1.7 1.7) (drill 1) (layers *.Cu *.Mask) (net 2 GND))
  (pad 8 thru_hole oval (at 2.54 7.62) (size 1.7 1.7) (drill 1) (layers *.Cu *.Mask) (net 2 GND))
  (pad 9 thru_hole oval (at 0 10.16) (size 1.7 1.7) (drill 1) (layers *.Cu *.Mask) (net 3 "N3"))
  (pad 10 thru_hole oval (at 2.54 10.16) (size 1.7 1.7) (drill 1) (layers *.Cu *.Mask) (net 3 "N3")))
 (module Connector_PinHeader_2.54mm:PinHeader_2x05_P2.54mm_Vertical (layer F.Cu) (at 190.5 99.06)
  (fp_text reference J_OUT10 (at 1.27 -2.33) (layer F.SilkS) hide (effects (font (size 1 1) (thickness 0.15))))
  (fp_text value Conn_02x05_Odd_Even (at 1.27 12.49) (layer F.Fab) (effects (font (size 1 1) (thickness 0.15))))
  (fp_line (start -1.33 -1.33) (end 0 -1.33) (layer F.SilkS) (width 0.12))
  (fp_line (start -1.33 0) (end -1.33 -1.33) (layer F.SilkS) (width 0.12))
  (fp_line (start 1.27 -1.33) (end 3.87 -1.33) (layer F.SilkS) (width 0.12))
  (fp_line (start 1.27 1.27) (end 1.27 -1.33) (layer F.SilkS) (width 0.12))
  (fp_line (start -1.33 1.27) (end 1.27 1.27) (layer F.SilkS) (width 0.12))
  (fp_line (start 3.87 -1.33) (end 3.87 11.49) (layer F.SilkS) (width 0.12))
  (fp_line (start -1.33 1.27) (end -1.33 11.49) (layer F.SilkS) (width 0.12))
  (fp_line (start -1.33 11.49) (end 3.87 11.49) (layer F.SilkS) (width 0.12))
  (pad 10 thru_hole oval (at 2.54 10.16) (size 1.7 1.7) (drill 1) (layers *.Cu *.Mask) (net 3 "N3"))
  (pad 9 thru_hole oval (at 0 10.16) (size 1.7 1.7) (drill 1) (layers *.Cu *.Mask) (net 3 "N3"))
  (pad 8 thru_hole oval (at 2.54 7.62) (size 1.7 1.7) (drill 1) (layers *.Cu *.Mask) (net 2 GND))
  (pad 7 thru_hole oval (at 0 7.62) (size 1.7 1.7) (drill 1) (layers *.Cu *.Mask) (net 2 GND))
  (pad 6 thru_hole oval (at 2.54 5.08) (size 1.7 1.7) (drill 1) (layers *.Cu *.Mask) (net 2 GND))
  (pad 5 thru_hole oval (at 0 5.08) (size 1.7 1.7) (drill 1) (layers *.Cu *.Mask) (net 2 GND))
  (pad 4 thru_hole oval (at 2.54 2.54) (size 1.7 1.7) (drill 1) (layers *.Cu *.Mask) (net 2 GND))
  (pad 3 thru_hole oval (at 0 2.54) (size 1.7 1.7) (drill 1) (layers *.Cu *.Mask) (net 2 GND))
  (pad 2 thru_hole oval (at 2.54 0) (size 1.7 1.7) (drill 1) (layers *.Cu *.Mask) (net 1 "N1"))
  (pad 1 thru_hole rect (at 0 0) (size 1.7 1.7) (drill 1) (layers *.Cu *.Mask) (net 1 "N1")))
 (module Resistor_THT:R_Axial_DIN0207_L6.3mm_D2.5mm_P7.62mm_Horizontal (layer F.Cu) (at 114.3 120.65 180)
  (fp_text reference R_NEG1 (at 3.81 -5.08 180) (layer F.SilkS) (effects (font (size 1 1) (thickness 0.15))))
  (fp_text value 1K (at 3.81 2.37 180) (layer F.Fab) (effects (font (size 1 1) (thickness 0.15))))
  (fp_line (start 0.54 -1.04) (end 0.54 -1.37) (layer F.SilkS) (width 0.12))
  (fp_line (start 0.54 -1.37) (end 7.08 -1.37) (layer F.SilkS) (width 0.12))
  (fp_line (start 7.08 -1.37) (end 7.08 -1.04) (layer F.SilkS) (width 0.12))
  (fp_line (start 0.54 1.04) (end 0.54 1.37) (layer F.SilkS) (width 0.12))
  (fp_line (start 0.54 1.37) (end 7.08 1.37) (layer F.SilkS) (width 0.12))
  (fp_line (start 7.08 1.37) (end 7.08 1.04) (layer F.SilkS) (width 0.12))
  (pad 1 thru_hole circle (at 0 0 180) (size 1.6 1.6) (drill 0.8) (layers *.Cu *.Mask) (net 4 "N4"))
  (pad 2 thru_hole oval (at 7.62 0 180) (size 1.6 1.6) (drill 0.8) (layers *.Cu *.Mask) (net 3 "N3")))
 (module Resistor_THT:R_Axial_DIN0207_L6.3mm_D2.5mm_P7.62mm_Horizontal (layer F.Cu) (at 132.08 88.9)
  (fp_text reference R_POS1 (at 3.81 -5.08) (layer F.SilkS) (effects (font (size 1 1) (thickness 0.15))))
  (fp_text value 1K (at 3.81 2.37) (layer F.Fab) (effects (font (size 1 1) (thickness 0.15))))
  (fp_line (start 7.08 1.37) (end 7.08 1.04) (layer F.SilkS) (width 0.12))
  (fp_line (start 0.54 1.37) (end 7.08 1.37) (layer F.SilkS) (width 0.12))
  (fp_line (start 0.54 1.04) (end 0.54 1.37) (layer F.SilkS) (width 0.12))
  (fp_line (start 7.08 -1.37) (end 7.08 -1.04) (layer F.SilkS) (width 0.12))
  (fp_line (start 0.54 -1.37) (end 7.08 -1.37) (layer F.SilkS) (width 0.12))
  (fp_line (start 0.54 -1.04) (end 0.54 -1.37) (layer F.SilkS) (width 0.12))
  (pad 2 thru_hole oval (at 7.62 0) (size 1.6 1.6) (drill 0.8) (layers *.Cu *.Mask) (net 2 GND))
  (pad 1 thru_hole circle (at 0 0) (size 1.6 1.6) (drill 0.8) (layers *.Cu *.Mask) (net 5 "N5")))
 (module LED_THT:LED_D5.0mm (layer F.Cu) (at 121.92 120.65)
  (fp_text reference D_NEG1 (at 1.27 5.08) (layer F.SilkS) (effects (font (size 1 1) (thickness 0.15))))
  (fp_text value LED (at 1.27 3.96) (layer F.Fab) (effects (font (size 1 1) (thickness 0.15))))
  (fp_line (start -1.29 -1.545) (end -1.29 1.545) (layer F.SilkS) (width 0.12))
  (fp_circle (center 1.27 0) (end 3.77 0) (layer F.SilkS) (width 0.12))
  (fp_arc (start 1.27 0) (end -1.29 1.54483) (angle -148.9) (layer F.SilkS) (width 0.12))
  (fp_arc (start 1.27 0) (end -1.29 -1.54483) (angle 148.9) (layer F.SilkS) (width 0.12))
  (pad 2 thru_hole circle (at 2.54 0) (size 1.8 1.8) (drill 0.9) (layers *.Cu *.Mask) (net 2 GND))
  (pad 1 thru_hole rect (at 0 0) (size 1.8 1.8) (drill 0.9) (layers *.Cu *.Mask) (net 4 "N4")))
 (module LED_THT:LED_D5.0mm (layer F.Cu) (at 124.46 88.9 180)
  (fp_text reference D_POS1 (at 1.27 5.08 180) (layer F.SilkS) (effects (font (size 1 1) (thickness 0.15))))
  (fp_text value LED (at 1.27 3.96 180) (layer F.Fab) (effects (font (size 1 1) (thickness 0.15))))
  (fp_arc (start 1.27 0) (end -1.29 -1.54483) (angle 148.9) (layer F.SilkS) (width 0.12))
  (fp_arc (start 1.27 0) (end -1.29 1.54483) (angle -148.9) (layer F.SilkS) (width 0.12))
  (fp_circle (center 1.27 0) (end 3.77 0) (layer F.SilkS) (width 0.12))
  (fp_line (start -1.29 -1.545) (end -1.29 1.545) (layer F.SilkS) (width 0.12))
  (pad 1 thru_hole rect (at 0 0 180) (size 1.8 1.8) (drill 0.9) (layers *.Cu *.Mask) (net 5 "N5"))
  (pad 2 thru_hole circle (at 2.54 0 180) (size 1.8 1.8) (drill 0.9) (layers *.Cu *.Mask) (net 1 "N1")))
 (gr_line (start 189.23 113.03) (end 194.31 113.03) (layer F.SilkS) (width 1))
 (gr_line (start 173.99 113.03) (end 179.07 113.03) (layer F.SilkS) (width 1))
 (gr_line (start 158.75 113.03) (end 163.83 113.03) (layer F.SilkS) (width 1))
 (gr_line (start 143.51 113.03) (end 148.59 113.03) (layer F.SilkS) (width 1))
 (gr_line (start 128.27 113.03) (end 133.35 113.03) (layer F.SilkS) (width 1))
 (gr_line (start 113.03 113.03) (end 118.11 113.03) (layer F.SilkS) (width 1))
 (gr_line (start 97.79 113.03) (end 102.87 113.03) (layer F.SilkS) (width 1))
 (gr_line (start 82.55 113.03) (end 87.63 113.03) (layer F.SilkS) (width 1))
 (gr_line (start 67.31 113.03) (end 72.39 113.03) (layer F.SilkS) (width 1))
 (gr_line (start 52.07 113.03) (end 57.15 113.03) (layer F.SilkS) (width 1))
 (gr_line (start 48.26 129.54) (end 48.26 78.74) (layer Edge.Cuts) (width 0.3))
 (gr_line (start 198.12 129.54) (end 48.26 129.54) (layer Edge.Cuts) (width 0.3))
 (gr_line (start 198.12 78.74) (end 198.12 129.54) (layer Edge.Cuts) (width 0.3))
 (gr_line (start 48.26 78.74) (end 198.12 78.74) (layer Edge.Cuts) (width 0.3))
 (segment (start 193.04 101.6) (end 53.34 101.6) (width 0.5) (layer F.Cu) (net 2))
 (segment (start 193.04 104.14) (end 53.34 104.14) (width 0.5) (layer F.Cu) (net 2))
 (segment (start 53.34 106.68) (end 193.04 106.68) (width 0.5) (layer F.Cu) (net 2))
 (segment (start 53.34 106.68) (end 53.34 101.6) (width 0.5) (layer F.Cu) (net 2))
 (segment (start 193.04 106.68) (end 193.04 101.6) (width 0.5) (layer F.Cu) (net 2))
 (segment (start 139.7 88.9) (end 193.04 88.9) (width 0.5) (layer F.Cu) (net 2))
 (segment (start 193.04 88.9) (end 195.58 91.44) (width 0.5) (layer F.Cu) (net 2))
 (segment (start 195.58 91.44) (end 195.58 101.6) (width 0.5) (layer F.Cu) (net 2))
 (segment (start 195.58 101.6) (end 193.04 101.6) (width 0.5) (layer F.Cu) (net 2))
 (segment (start 195.58 114.3) (end 195.58 106.68) (width 0.5) (layer F.Cu) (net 2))
 (segment (start 189.23 120.65) (end 195.58 114.3) (width 0.5) (layer F.Cu) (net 2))
 (segment (start 195.58 106.68) (end 193.04 106.68) (width 0.5) (layer F.Cu) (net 2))
 (segment (start 124.46 120.65) (end 189.23 120.65) (width 0.5) (layer F.Cu) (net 2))
 (segment (start 114.3 120.65) (end 121.92 120.65) (width 0.5) (layer F.Cu) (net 4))
 (segment (start 124.46 88.9) (end 132.08 88.9) (width 0.5) (layer F.Cu) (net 5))
 (segment (start 53.34 99.06) (end 193.04 99.06) (width 0.5) (layer F.Cu) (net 1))
 (segment (start 116.84 91.44) (end 119.38 88.9) (width 0.5) (layer F.Cu) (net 1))
 (segment (start 119.38 88.9) (end 121.92 88.9) (width 0.5) (layer F.Cu) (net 1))
 (segment (start 116.84 99.06) (end 116.84 91.44) (width 0.5) (layer F.Cu) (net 1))
 (segment (start 193.04 109.22) (end 53.34 109.22) (width 0.5) (layer F.Cu) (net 3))
 (segment (start 106.68 120.65) (end 105.41 120.65) (width 0.5) (layer F.Cu) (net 3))
 (segment (start 101.6 116.84) (end 101.6 109.22) (width 0.5) (layer F.Cu) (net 3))
 (segment (start 105.41 120.65) (end 101.6 116.84) (width 0.5) (layer F.Cu) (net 3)))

